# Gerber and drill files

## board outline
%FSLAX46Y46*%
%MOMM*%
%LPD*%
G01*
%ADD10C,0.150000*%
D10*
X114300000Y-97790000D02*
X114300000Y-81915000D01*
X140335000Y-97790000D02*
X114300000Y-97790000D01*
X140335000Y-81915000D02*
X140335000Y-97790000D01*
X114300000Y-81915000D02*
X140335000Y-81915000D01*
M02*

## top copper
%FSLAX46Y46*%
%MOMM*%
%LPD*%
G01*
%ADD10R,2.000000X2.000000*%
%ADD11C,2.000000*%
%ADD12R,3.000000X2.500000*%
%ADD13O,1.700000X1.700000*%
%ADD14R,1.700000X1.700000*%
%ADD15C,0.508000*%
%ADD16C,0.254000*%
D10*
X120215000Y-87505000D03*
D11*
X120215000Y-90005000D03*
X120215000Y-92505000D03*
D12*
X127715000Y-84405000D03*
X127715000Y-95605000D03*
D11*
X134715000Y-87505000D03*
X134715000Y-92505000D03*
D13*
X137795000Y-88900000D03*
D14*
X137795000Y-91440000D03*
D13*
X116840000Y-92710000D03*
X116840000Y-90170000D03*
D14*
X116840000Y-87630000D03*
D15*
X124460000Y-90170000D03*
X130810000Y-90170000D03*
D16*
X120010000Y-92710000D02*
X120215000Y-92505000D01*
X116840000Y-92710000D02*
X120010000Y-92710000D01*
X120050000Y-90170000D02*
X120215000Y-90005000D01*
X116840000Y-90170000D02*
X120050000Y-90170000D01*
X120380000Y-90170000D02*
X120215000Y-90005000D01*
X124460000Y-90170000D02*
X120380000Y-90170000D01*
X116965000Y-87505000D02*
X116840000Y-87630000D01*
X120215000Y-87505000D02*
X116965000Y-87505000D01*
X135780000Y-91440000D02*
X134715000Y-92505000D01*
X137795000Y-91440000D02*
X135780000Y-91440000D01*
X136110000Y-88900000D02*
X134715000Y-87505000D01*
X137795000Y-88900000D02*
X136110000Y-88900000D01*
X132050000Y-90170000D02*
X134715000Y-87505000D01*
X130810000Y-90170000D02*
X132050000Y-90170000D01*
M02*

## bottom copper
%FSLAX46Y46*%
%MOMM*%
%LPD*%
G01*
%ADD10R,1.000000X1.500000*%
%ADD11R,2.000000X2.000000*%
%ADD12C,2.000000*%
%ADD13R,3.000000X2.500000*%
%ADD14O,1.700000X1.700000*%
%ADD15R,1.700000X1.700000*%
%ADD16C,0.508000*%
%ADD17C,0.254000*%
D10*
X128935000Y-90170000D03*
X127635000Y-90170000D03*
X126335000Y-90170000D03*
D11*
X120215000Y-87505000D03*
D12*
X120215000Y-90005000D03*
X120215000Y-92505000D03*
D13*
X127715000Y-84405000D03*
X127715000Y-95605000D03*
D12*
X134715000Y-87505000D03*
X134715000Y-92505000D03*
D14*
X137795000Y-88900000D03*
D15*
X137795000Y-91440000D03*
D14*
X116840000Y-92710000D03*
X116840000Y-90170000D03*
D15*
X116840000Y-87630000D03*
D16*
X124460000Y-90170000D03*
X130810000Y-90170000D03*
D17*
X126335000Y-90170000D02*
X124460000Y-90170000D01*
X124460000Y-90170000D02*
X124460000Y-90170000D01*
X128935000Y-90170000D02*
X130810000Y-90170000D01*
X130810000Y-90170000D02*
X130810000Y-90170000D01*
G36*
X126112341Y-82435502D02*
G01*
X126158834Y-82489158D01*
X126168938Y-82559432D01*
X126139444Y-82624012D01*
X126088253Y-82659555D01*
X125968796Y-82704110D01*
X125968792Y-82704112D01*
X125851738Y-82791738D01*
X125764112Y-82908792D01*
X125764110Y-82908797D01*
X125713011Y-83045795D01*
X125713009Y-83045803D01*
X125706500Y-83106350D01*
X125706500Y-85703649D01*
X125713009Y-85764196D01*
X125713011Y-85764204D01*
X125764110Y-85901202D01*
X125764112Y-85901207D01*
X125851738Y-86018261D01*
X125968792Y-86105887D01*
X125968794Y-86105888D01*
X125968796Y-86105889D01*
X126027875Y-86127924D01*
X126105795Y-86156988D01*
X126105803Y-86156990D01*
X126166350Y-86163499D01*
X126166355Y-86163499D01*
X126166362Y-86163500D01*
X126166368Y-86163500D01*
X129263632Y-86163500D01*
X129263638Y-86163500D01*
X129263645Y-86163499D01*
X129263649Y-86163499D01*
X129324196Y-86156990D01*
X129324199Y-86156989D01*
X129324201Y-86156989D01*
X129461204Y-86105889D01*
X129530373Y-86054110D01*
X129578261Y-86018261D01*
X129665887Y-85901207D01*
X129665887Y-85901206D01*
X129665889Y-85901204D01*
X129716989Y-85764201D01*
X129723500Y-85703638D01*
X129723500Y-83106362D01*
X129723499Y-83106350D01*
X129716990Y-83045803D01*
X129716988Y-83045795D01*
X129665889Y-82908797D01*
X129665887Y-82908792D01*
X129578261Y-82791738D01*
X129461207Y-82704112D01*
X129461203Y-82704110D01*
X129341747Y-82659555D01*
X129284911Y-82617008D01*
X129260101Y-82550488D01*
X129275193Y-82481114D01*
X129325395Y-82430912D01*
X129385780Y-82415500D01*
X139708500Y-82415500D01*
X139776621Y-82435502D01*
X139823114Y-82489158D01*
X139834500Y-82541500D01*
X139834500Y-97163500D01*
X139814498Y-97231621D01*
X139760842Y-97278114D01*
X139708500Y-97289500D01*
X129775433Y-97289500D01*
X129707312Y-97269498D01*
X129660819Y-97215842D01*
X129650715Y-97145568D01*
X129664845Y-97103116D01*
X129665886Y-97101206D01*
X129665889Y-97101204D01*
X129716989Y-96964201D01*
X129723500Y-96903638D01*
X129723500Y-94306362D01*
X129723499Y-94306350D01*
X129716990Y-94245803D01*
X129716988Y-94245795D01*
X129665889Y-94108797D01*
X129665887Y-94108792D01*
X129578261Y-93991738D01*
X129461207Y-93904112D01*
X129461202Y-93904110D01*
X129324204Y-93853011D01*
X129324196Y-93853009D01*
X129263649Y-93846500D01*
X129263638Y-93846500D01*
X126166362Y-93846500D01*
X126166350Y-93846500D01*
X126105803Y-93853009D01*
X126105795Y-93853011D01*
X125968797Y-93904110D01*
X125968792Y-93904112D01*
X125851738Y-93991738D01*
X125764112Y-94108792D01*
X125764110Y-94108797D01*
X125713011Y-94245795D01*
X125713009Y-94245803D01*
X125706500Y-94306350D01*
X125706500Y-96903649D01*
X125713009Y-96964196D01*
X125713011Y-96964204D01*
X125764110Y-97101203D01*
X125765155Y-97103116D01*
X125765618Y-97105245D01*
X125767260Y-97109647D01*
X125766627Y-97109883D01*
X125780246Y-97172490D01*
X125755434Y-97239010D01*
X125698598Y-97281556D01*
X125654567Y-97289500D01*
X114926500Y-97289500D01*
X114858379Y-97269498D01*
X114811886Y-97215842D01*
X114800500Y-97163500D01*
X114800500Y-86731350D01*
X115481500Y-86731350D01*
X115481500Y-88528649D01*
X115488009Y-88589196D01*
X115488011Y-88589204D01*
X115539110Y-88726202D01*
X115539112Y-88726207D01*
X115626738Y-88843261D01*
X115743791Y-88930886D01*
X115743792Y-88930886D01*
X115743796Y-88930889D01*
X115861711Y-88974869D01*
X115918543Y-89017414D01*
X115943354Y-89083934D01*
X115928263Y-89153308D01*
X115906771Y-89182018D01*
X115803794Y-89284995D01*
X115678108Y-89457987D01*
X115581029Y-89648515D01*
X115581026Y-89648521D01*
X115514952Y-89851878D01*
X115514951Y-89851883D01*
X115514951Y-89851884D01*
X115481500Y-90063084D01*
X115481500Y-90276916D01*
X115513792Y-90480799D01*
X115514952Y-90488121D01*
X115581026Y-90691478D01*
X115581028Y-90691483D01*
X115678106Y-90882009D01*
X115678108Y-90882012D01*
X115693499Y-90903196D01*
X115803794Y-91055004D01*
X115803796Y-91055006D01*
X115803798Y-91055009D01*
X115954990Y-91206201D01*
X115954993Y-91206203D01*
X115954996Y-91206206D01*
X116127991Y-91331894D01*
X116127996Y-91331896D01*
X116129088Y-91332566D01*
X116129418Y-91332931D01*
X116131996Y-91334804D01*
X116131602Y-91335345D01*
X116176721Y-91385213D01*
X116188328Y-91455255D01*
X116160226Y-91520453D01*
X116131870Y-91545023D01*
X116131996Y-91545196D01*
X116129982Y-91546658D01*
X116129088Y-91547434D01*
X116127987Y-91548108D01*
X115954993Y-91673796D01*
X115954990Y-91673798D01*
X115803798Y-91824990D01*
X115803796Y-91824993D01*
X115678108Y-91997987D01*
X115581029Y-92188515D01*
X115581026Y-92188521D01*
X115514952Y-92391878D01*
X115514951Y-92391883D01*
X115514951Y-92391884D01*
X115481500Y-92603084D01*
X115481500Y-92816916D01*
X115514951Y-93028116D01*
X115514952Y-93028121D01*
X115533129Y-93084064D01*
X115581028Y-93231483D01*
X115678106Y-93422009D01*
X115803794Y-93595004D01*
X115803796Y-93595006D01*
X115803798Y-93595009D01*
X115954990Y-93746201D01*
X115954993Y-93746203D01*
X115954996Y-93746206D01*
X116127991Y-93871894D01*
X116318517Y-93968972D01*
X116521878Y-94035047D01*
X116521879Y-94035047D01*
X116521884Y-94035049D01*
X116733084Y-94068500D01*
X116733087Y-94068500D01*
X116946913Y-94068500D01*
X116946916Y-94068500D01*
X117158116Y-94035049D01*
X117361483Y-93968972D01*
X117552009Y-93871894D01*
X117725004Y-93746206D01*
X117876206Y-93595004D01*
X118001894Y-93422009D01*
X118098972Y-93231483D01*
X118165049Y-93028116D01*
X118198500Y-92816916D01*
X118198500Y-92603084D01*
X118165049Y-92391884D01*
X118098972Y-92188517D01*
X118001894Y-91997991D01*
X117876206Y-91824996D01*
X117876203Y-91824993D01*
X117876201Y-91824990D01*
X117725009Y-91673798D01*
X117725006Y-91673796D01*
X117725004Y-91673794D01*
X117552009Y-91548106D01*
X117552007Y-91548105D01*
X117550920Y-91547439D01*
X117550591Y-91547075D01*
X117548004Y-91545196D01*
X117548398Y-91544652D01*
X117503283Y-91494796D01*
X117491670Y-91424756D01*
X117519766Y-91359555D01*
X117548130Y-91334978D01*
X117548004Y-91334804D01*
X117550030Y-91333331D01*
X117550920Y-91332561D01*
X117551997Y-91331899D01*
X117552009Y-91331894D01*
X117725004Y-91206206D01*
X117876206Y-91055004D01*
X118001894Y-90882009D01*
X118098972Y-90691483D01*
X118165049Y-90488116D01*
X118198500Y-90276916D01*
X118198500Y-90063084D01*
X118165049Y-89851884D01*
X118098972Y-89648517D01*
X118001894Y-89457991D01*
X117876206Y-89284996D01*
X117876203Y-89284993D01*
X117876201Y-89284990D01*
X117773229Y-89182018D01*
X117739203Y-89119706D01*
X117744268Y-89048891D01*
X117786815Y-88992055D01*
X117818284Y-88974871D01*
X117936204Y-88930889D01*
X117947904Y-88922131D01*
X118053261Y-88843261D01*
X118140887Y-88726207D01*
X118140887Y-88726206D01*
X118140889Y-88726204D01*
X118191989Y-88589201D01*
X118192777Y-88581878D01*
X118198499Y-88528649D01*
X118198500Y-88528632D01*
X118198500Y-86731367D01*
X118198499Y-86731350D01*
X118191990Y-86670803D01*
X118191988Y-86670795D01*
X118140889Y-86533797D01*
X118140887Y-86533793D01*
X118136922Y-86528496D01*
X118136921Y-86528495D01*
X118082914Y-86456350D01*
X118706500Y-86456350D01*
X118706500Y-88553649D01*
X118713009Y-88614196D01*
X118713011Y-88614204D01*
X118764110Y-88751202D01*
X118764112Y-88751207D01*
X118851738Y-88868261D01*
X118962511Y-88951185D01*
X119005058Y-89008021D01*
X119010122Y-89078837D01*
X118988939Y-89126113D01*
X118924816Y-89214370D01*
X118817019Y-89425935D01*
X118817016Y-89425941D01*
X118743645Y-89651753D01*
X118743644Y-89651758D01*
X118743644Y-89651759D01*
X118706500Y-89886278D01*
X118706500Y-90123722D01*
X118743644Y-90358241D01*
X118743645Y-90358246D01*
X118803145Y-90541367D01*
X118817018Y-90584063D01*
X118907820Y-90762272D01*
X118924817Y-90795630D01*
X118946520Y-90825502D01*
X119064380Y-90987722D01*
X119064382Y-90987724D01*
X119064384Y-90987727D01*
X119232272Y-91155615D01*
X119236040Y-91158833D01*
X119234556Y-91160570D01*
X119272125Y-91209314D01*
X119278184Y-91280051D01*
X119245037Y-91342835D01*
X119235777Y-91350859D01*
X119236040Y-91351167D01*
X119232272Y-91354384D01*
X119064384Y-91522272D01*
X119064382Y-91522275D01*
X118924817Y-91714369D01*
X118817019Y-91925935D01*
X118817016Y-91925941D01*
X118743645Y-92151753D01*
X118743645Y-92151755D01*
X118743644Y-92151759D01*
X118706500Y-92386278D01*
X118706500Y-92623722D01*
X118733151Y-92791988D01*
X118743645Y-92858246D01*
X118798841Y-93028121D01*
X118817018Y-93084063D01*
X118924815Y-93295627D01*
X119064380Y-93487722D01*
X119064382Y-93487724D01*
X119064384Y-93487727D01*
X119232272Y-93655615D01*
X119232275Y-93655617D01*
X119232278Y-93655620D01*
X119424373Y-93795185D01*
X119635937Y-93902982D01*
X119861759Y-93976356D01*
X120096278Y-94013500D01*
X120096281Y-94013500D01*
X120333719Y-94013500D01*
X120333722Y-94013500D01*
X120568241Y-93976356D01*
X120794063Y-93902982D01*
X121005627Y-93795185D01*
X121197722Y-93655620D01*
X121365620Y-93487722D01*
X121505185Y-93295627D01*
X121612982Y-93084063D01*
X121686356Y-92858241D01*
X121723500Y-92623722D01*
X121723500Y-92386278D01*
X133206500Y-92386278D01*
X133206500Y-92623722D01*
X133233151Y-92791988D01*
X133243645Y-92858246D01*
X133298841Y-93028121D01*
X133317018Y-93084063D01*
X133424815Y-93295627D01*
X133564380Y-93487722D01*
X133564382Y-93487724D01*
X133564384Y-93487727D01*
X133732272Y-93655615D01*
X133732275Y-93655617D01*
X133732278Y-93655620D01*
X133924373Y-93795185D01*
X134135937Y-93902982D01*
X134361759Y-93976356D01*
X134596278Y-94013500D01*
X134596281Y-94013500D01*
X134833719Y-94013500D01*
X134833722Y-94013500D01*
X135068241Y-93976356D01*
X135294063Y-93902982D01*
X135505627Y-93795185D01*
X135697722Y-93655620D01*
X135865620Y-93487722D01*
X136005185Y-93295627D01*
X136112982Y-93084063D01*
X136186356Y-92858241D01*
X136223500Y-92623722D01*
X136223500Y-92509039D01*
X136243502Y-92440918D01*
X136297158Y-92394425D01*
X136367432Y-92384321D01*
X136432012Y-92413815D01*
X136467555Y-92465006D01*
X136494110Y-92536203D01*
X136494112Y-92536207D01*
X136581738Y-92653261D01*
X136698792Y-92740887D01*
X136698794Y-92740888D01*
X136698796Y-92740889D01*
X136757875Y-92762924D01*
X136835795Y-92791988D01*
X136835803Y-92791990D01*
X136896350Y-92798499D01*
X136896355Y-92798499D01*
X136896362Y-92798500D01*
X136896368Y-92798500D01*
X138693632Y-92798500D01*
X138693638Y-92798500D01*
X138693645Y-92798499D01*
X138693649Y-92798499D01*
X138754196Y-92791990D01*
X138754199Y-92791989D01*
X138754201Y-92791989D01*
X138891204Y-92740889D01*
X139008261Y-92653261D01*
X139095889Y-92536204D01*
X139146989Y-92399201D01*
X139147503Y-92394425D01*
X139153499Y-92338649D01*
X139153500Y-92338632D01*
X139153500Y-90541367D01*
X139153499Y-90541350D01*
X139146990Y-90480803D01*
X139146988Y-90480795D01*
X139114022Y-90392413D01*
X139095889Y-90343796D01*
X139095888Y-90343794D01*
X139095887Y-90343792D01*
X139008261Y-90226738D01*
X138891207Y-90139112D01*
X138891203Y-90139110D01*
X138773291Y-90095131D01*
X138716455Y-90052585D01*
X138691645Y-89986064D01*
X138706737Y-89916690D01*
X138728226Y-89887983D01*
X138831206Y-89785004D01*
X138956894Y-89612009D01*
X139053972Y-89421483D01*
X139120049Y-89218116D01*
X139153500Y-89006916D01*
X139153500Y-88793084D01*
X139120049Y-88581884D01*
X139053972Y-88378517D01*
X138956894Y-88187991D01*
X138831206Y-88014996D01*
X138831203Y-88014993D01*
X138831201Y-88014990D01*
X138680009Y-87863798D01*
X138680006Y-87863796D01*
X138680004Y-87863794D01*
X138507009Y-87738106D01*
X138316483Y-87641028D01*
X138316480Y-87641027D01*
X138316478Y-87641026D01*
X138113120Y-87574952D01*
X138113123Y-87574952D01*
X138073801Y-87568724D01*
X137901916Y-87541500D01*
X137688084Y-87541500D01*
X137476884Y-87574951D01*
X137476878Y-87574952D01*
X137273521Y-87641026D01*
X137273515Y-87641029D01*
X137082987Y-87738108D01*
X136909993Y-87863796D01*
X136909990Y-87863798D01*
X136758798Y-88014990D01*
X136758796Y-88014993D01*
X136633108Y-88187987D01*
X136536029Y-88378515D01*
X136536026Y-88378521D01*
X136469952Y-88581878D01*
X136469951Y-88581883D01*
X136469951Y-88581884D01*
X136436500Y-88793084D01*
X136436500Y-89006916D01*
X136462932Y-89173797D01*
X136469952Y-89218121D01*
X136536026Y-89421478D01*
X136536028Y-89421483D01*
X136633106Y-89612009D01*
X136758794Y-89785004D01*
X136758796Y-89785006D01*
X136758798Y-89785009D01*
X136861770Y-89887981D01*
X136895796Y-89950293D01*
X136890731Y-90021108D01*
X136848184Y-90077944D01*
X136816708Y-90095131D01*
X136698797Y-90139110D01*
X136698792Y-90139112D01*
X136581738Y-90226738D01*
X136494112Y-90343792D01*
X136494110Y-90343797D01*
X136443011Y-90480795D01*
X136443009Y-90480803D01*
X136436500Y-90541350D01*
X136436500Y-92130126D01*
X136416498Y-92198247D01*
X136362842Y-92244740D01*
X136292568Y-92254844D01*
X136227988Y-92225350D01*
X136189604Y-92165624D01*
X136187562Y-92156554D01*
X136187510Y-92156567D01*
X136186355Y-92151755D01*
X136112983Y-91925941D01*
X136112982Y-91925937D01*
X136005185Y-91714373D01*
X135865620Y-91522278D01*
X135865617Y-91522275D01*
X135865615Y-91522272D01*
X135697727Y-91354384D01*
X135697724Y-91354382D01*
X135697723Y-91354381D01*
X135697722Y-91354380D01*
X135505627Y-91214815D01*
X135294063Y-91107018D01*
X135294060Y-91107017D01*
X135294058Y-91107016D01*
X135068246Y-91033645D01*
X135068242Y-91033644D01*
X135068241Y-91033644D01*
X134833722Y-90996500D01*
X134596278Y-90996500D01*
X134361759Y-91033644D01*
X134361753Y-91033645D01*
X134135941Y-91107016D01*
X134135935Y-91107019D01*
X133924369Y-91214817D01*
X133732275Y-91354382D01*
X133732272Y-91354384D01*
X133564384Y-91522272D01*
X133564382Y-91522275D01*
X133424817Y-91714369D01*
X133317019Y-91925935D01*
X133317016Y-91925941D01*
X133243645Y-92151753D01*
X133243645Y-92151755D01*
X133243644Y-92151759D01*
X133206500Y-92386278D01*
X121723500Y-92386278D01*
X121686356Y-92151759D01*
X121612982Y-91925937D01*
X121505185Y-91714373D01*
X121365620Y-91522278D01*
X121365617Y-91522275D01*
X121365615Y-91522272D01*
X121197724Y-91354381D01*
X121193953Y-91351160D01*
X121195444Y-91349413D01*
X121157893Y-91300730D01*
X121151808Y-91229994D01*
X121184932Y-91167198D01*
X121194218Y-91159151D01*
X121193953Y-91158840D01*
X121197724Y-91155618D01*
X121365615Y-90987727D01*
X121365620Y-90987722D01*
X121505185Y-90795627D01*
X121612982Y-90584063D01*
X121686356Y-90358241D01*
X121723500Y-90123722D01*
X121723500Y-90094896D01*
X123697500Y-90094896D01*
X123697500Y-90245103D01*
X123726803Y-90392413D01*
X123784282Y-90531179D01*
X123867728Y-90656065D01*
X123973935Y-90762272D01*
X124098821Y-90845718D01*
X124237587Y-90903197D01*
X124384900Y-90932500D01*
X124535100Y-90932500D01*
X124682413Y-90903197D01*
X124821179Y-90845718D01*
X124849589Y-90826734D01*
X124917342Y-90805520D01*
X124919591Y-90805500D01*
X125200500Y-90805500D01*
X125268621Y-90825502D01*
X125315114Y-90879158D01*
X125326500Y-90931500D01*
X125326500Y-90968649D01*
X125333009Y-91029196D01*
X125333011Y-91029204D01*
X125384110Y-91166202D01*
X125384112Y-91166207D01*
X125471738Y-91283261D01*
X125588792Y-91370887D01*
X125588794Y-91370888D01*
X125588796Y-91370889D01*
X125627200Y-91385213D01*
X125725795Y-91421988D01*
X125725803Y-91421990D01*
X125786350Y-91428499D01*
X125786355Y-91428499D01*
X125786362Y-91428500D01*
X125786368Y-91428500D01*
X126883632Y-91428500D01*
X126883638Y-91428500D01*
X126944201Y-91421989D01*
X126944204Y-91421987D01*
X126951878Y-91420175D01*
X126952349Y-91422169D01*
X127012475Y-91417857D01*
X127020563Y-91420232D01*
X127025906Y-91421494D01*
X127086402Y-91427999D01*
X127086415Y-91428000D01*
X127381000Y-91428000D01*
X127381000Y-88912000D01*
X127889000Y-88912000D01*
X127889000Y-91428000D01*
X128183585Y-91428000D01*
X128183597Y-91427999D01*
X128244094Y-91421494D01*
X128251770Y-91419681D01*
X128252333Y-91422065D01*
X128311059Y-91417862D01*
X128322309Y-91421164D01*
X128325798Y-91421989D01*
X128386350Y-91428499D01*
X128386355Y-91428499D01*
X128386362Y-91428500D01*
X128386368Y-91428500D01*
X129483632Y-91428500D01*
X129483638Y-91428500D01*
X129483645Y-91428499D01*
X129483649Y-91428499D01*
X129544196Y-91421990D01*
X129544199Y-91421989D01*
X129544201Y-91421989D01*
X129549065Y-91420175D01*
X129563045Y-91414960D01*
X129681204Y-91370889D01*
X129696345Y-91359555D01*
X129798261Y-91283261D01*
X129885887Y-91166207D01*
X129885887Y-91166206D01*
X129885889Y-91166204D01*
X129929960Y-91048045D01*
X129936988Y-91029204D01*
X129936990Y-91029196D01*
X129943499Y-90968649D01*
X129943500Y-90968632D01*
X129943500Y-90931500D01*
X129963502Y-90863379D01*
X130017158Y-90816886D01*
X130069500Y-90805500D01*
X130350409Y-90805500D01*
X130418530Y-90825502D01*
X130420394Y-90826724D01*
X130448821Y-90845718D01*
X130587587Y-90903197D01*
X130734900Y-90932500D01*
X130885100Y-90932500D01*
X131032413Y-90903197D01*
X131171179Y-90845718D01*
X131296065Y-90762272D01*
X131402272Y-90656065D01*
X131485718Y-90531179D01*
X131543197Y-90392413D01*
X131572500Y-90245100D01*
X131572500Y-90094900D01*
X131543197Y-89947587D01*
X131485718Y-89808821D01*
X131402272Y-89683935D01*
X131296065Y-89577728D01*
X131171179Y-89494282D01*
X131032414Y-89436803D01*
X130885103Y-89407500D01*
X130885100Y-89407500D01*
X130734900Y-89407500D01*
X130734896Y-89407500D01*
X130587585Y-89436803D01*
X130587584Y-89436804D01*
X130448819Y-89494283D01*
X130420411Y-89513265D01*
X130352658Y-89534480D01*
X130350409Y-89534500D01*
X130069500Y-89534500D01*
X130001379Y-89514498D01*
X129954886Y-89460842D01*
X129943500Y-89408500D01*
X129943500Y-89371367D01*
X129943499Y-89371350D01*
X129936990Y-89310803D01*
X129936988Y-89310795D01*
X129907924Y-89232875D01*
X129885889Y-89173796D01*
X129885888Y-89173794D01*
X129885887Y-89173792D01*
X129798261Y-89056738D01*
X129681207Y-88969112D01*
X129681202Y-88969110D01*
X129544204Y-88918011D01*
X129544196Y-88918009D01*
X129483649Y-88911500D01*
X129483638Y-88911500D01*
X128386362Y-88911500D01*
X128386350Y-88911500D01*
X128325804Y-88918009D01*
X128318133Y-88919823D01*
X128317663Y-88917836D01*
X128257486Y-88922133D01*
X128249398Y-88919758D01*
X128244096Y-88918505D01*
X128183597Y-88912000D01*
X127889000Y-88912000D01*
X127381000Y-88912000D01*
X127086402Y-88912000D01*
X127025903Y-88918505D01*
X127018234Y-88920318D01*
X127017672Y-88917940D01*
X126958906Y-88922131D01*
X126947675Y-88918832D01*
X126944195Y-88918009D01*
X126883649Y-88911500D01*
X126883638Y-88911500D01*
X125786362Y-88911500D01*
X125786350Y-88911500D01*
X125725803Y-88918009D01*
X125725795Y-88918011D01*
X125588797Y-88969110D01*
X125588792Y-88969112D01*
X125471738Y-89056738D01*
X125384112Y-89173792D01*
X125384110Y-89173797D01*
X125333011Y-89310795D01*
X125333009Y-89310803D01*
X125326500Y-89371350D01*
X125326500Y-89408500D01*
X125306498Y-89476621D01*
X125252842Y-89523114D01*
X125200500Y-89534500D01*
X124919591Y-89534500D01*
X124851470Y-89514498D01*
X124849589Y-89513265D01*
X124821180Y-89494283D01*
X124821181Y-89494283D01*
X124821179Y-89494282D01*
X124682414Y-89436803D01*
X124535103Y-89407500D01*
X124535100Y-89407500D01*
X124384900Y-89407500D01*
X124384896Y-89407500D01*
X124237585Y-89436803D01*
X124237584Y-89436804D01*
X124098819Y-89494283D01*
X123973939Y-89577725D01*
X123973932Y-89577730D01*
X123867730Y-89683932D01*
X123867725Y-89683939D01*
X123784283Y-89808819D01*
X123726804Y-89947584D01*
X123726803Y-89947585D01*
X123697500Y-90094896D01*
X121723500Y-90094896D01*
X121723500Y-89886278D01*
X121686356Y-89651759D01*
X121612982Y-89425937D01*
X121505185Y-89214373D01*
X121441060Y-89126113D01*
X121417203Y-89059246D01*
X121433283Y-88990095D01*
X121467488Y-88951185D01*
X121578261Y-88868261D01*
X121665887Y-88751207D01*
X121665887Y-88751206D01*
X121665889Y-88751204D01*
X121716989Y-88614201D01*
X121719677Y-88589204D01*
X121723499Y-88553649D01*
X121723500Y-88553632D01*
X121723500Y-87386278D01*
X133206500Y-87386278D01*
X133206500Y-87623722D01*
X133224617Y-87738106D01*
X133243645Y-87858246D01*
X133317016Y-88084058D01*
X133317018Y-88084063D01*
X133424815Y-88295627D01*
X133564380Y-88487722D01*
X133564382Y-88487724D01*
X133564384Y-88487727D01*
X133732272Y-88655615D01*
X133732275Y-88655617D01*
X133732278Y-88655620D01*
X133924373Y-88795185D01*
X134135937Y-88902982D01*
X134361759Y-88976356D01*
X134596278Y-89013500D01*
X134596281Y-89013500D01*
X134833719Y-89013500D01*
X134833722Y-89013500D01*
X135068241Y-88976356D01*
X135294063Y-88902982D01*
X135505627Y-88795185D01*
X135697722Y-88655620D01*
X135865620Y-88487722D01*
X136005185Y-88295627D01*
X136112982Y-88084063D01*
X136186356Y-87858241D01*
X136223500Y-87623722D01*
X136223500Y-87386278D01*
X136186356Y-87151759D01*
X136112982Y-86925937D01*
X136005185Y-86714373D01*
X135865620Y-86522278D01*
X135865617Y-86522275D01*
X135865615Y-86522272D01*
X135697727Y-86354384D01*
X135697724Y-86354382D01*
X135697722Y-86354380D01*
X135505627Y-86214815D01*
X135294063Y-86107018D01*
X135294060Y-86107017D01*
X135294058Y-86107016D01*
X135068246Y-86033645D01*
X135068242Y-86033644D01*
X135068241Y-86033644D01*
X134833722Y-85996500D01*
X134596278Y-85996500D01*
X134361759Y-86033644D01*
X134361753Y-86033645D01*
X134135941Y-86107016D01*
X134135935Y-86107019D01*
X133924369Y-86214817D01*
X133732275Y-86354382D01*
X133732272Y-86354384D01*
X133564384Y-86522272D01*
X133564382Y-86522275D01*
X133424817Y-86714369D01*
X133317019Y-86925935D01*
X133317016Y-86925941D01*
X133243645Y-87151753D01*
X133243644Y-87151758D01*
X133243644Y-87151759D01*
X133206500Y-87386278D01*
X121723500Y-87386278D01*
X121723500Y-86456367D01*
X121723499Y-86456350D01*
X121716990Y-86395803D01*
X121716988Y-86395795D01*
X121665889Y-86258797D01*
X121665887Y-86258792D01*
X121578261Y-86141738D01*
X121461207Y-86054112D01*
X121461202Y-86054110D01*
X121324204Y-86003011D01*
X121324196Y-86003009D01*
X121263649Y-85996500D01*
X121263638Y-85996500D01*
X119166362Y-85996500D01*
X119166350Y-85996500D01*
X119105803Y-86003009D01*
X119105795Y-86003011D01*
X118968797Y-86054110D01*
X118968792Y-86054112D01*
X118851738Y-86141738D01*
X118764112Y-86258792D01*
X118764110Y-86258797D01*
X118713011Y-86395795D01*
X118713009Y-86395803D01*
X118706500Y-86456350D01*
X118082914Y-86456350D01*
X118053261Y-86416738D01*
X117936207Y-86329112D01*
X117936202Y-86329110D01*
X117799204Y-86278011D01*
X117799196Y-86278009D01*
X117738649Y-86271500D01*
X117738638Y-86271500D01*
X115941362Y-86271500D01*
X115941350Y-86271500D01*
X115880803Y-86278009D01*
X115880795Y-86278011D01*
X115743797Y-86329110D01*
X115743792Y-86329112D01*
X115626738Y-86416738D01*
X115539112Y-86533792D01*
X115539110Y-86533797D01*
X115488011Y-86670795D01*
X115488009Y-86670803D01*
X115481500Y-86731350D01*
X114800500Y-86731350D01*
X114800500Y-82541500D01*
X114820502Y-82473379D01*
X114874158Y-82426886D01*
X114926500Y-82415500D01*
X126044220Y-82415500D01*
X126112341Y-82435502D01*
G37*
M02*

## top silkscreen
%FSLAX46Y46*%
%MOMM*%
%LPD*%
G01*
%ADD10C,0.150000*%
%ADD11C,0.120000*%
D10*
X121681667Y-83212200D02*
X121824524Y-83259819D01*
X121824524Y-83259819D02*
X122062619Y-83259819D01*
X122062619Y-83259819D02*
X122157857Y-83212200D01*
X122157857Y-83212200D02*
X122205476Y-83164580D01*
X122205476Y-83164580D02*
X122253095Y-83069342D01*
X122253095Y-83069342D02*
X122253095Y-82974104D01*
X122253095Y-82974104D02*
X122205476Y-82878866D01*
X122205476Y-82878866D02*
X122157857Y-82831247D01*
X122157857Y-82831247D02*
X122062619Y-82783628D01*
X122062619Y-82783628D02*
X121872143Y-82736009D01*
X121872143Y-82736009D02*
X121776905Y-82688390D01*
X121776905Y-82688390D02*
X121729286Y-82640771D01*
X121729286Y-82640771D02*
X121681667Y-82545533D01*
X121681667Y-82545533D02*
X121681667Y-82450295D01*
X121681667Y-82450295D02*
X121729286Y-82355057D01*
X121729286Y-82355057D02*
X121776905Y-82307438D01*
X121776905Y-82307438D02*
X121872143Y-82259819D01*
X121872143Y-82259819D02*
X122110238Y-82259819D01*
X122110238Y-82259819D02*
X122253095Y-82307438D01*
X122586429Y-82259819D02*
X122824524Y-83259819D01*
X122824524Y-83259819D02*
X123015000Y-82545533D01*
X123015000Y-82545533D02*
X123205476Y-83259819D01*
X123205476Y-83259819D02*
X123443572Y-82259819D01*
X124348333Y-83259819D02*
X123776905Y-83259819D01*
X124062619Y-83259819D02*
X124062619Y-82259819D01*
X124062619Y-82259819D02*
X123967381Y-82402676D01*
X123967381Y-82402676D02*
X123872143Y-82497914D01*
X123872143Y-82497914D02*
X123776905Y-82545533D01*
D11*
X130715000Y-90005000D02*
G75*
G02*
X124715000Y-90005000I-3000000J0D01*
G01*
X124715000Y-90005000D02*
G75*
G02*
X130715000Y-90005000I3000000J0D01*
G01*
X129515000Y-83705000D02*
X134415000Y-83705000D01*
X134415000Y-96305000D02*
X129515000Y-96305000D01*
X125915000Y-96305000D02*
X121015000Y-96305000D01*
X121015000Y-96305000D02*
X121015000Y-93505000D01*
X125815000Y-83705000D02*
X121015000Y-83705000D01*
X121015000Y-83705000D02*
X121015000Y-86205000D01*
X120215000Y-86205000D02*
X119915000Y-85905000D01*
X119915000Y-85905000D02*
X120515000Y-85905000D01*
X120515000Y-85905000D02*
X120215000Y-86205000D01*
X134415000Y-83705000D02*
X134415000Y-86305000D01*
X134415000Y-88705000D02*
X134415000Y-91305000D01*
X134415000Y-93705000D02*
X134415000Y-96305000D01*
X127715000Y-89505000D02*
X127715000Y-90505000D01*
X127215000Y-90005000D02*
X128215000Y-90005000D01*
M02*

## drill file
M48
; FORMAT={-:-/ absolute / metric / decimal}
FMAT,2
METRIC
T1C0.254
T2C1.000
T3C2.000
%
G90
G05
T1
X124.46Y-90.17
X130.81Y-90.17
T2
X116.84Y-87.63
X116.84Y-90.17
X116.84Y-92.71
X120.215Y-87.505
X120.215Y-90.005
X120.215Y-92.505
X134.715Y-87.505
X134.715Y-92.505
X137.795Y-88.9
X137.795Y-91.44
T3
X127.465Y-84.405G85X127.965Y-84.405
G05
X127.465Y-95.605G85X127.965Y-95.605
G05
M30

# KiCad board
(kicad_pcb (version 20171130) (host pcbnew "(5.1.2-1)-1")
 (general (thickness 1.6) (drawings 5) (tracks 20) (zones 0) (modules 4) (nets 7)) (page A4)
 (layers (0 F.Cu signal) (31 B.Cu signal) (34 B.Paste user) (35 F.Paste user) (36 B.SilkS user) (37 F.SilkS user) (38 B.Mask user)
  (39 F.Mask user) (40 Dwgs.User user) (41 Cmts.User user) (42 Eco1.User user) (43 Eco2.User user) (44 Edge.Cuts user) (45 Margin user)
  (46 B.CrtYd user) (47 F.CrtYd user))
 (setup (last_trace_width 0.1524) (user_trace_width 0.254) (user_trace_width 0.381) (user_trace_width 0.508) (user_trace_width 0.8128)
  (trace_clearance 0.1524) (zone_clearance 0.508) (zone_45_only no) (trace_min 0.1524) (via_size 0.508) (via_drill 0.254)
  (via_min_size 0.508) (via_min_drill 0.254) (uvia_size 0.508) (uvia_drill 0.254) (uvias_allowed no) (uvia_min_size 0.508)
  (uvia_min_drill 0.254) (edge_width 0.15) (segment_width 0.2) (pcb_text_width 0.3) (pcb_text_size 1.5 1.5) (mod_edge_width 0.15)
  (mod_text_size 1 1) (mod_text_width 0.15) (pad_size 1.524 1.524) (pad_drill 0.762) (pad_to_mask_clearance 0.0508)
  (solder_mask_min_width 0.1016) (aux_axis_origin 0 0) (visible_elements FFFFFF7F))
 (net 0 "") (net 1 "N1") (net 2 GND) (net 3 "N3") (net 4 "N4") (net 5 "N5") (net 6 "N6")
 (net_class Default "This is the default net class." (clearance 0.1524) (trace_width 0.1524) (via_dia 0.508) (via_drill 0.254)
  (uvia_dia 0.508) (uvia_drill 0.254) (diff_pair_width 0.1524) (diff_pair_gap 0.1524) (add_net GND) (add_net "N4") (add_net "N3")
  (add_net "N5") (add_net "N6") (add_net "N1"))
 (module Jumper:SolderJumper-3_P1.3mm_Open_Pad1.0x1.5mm (layer B.Cu) (at 127.635 90.17 180)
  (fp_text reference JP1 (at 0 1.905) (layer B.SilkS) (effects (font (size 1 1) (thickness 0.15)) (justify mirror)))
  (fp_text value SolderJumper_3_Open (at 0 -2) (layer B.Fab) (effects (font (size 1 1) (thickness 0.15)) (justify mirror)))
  (pad 1 smd rect (at -1.3 0 180) (size 1 1.5) (layers B.Cu B.Mask) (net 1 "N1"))
  (pad 2 smd rect (at 0 0 180) (size 1 1.5) (layers B.Cu B.Mask) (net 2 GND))
  (pad 3 smd rect (at 1.3 0 180) (size 1 1.5) (layers B.Cu B.Mask) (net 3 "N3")))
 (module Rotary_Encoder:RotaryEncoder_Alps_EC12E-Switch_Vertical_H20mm (layer F.Cu) (at 120.215 87.505)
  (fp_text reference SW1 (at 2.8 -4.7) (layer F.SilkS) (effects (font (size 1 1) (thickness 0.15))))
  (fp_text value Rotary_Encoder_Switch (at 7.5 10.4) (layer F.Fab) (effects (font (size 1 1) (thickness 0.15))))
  (fp_circle (center 7.5 2.5) (end 10.5 2.5) (layer F.SilkS) (width 0.12))
  (fp_line (start 9.3 -3.8) (end 14.2 -3.8) (layer F.SilkS) (width 0.12))
  (fp_line (start 14.2 8.8) (end 9.3 8.8) (layer F.SilkS) (width 0.12))
  (fp_line (start 5.7 8.8) (end 0.8 8.8) (layer F.SilkS) (width 0.12))
  (fp_line (start 0.8 8.8) (end 0.8 6) (layer F.SilkS) (width 0.12))
  (fp_line (start 5.6 -3.8) (end 0.8 -3.8) (layer F.SilkS) (width 0.12))
  (fp_line (start 0.8 -3.8) (end 0.8 -1.3) (layer F.SilkS) (width 0.12))
  (fp_line (start 0 -1.3) (end -0.3 -1.6) (layer F.SilkS) (width 0.12))
  (fp_line (start -0.3 -1.6) (end 0.3 -1.6) (layer F.SilkS) (width 0.12))
  (fp_line (start 0.3 -1.6) (end 0 -1.3) (layer F.SilkS) (width 0.12))
  (fp_line (start 14.2 -3.8) (end 14.2 -1.2) (layer F.SilkS) (width 0.12))
  (fp_line (start 14.2 1.2) (end 14.2 3.8) (layer F.SilkS) (width 0.12))
  (fp_line (start 14.2 6.2) (end 14.2 8.8) (layer F.SilkS) (width 0.12))
  (fp_line (start 7.5 2) (end 7.5 3) (layer F.SilkS) (width 0.12))
  (fp_line (start 7 2.5) (end 8 2.5) (layer F.SilkS) (width 0.12))
  (pad A thru_hole rect (at 0 0) (size 2 2) (drill 1) (layers *.Cu *.Mask) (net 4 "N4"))
  (pad C thru_hole circle (at 0 2.5) (size 2 2) (drill 1) (layers *.Cu *.Mask) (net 3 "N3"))
  (pad B thru_hole circle (at 0 5) (size 2 2) (drill 1) (layers *.Cu *.Mask) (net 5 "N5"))
  (pad MP thru_hole rect (at 7.5 -3.1) (size 3 2.5) (drill oval 2.5 2) (layers *.Cu *.Mask))
  (pad MP thru_hole rect (at 7.5 8.1) (size 3 2.5) (drill oval 2.5 2) (layers *.Cu *.Mask))
  (pad S1 thru_hole circle (at 14.5 0) (size 2 2) (drill 1) (layers *.Cu *.Mask) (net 1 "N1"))
  (pad S2 thru_hole circle (at 14.5 5) (size 2 2) (drill 1) (layers *.Cu *.Mask) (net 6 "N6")))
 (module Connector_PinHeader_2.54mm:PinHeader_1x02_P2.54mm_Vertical (layer B.Cu) (at 137.795 91.44)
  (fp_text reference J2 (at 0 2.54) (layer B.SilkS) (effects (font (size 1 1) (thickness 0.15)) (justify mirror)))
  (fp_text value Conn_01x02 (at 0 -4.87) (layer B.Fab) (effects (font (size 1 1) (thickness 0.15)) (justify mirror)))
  (pad 2 thru_hole oval (at 0 -2.54) (size 1.7 1.7) (drill 1) (layers *.Cu *.Mask) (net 1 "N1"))
  (pad 1 thru_hole rect (at 0 0) (size 1.7 1.7) (drill 1) (layers *.Cu *.Mask) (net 6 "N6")))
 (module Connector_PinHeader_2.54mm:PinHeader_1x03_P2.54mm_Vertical (layer B.Cu) (at 116.84 87.63 180)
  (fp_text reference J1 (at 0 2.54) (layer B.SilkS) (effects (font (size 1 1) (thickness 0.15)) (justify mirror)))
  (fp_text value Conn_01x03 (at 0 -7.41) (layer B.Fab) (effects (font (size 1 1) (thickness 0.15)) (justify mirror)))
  (pad 3 thru_hole oval (at 0 -5.08 180) (size 1.7 1.7) (drill 1) (layers *.Cu *.Mask) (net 5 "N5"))
  (pad 2 thru_hole oval (at 0 -2.54 180) (size 1.7 1.7) (drill 1) (layers *.Cu *.Mask) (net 3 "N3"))
  (pad 1 thru_hole rect (at 0 0 180) (size 1.7 1.7) (drill 1) (layers *.Cu *.Mask) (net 4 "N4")))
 (gr_line (start 114.3 97.79) (end 114.3 81.915) (layer Edge.Cuts) (width 0.15))
 (gr_line (start 140.335 97.79) (end 114.3 97.79) (layer Edge.Cuts) (width 0.15))
 (gr_line (start 140.335 81.915) (end 140.335 97.79) (layer Edge.Cuts) (width 0.15))
 (gr_line (start 114.3 81.915) (end 140.335 81.915) (layer Edge.Cuts) (width 0.15))
 (segment (start 120.01 92.71) (end 120.215 92.505) (width 0.254) (layer F.Cu) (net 5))
 (segment (start 116.84 92.71) (end 120.01 92.71) (width 0.254) (layer F.Cu) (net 5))
 (segment (start 120.05 90.17) (end 120.215 90.005) (width 0.254) (layer F.Cu) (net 3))
 (segment (start 116.84 90.17) (end 120.05 90.17) (width 0.254) (layer F.Cu) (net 3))
 (segment (start 126.335 90.17) (end 124.46 90.17) (width 0.254) (layer B.Cu) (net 3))
 (segment (start 124.46 90.17) (end 124.46 90.17) (width 0.254) (layer B.Cu) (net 3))
 (via (at 124.46 90.17) (size 0.508) (drill 0.254) (layers F.Cu B.Cu) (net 3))
 (segment (start 120.38 90.17) (end 120.215 90.005) (width 0.254) (layer F.Cu) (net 3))
 (segment (start 124.46 90.17) (end 120.38 90.17) (width 0.254) (layer F.Cu) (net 3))
 (segment (start 116.965 87.505) (end 116.84 87.63) (width 0.254) (layer F.Cu) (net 4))
 (segment (start 120.215 87.505) (end 116.965 87.505) (width 0.254) (layer F.Cu) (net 4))
 (segment (start 135.78 91.44) (end 134.715 92.505) (width 0.254) (layer F.Cu) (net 6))
 (segment (start 137.795 91.44) (end 135.78 91.44) (width 0.254) (layer F.Cu) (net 6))
 (segment (start 136.11 88.9) (end 134.715 87.505) (width 0.254) (layer F.Cu) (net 1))
 (segment (start 137.795 88.9) (end 136.11 88.9) (width 0.254) (layer F.Cu) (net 1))
 (segment (start 128.935 90.17) (end 130.81 90.17) (width 0.254) (layer B.Cu) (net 1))
 (segment (start 130.81 90.17) (end 130.81 90.17) (width 0.254) (layer B.Cu) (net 1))
 (via (at 130.81 90.17) (size 0.508) (drill 0.254) (layers F.Cu B.Cu) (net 1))
 (segment (start 132.05 90.17) (end 134.715 87.505) (width 0.254) (layer F.Cu) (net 1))
 (segment (start 130.81 90.17) (end 132.05 90.17) (width 0.254) (layer F.Cu) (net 1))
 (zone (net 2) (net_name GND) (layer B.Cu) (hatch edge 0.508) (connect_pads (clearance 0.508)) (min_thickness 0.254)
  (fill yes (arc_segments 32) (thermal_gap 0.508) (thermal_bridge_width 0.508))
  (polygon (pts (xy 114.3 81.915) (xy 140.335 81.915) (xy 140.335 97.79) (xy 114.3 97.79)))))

